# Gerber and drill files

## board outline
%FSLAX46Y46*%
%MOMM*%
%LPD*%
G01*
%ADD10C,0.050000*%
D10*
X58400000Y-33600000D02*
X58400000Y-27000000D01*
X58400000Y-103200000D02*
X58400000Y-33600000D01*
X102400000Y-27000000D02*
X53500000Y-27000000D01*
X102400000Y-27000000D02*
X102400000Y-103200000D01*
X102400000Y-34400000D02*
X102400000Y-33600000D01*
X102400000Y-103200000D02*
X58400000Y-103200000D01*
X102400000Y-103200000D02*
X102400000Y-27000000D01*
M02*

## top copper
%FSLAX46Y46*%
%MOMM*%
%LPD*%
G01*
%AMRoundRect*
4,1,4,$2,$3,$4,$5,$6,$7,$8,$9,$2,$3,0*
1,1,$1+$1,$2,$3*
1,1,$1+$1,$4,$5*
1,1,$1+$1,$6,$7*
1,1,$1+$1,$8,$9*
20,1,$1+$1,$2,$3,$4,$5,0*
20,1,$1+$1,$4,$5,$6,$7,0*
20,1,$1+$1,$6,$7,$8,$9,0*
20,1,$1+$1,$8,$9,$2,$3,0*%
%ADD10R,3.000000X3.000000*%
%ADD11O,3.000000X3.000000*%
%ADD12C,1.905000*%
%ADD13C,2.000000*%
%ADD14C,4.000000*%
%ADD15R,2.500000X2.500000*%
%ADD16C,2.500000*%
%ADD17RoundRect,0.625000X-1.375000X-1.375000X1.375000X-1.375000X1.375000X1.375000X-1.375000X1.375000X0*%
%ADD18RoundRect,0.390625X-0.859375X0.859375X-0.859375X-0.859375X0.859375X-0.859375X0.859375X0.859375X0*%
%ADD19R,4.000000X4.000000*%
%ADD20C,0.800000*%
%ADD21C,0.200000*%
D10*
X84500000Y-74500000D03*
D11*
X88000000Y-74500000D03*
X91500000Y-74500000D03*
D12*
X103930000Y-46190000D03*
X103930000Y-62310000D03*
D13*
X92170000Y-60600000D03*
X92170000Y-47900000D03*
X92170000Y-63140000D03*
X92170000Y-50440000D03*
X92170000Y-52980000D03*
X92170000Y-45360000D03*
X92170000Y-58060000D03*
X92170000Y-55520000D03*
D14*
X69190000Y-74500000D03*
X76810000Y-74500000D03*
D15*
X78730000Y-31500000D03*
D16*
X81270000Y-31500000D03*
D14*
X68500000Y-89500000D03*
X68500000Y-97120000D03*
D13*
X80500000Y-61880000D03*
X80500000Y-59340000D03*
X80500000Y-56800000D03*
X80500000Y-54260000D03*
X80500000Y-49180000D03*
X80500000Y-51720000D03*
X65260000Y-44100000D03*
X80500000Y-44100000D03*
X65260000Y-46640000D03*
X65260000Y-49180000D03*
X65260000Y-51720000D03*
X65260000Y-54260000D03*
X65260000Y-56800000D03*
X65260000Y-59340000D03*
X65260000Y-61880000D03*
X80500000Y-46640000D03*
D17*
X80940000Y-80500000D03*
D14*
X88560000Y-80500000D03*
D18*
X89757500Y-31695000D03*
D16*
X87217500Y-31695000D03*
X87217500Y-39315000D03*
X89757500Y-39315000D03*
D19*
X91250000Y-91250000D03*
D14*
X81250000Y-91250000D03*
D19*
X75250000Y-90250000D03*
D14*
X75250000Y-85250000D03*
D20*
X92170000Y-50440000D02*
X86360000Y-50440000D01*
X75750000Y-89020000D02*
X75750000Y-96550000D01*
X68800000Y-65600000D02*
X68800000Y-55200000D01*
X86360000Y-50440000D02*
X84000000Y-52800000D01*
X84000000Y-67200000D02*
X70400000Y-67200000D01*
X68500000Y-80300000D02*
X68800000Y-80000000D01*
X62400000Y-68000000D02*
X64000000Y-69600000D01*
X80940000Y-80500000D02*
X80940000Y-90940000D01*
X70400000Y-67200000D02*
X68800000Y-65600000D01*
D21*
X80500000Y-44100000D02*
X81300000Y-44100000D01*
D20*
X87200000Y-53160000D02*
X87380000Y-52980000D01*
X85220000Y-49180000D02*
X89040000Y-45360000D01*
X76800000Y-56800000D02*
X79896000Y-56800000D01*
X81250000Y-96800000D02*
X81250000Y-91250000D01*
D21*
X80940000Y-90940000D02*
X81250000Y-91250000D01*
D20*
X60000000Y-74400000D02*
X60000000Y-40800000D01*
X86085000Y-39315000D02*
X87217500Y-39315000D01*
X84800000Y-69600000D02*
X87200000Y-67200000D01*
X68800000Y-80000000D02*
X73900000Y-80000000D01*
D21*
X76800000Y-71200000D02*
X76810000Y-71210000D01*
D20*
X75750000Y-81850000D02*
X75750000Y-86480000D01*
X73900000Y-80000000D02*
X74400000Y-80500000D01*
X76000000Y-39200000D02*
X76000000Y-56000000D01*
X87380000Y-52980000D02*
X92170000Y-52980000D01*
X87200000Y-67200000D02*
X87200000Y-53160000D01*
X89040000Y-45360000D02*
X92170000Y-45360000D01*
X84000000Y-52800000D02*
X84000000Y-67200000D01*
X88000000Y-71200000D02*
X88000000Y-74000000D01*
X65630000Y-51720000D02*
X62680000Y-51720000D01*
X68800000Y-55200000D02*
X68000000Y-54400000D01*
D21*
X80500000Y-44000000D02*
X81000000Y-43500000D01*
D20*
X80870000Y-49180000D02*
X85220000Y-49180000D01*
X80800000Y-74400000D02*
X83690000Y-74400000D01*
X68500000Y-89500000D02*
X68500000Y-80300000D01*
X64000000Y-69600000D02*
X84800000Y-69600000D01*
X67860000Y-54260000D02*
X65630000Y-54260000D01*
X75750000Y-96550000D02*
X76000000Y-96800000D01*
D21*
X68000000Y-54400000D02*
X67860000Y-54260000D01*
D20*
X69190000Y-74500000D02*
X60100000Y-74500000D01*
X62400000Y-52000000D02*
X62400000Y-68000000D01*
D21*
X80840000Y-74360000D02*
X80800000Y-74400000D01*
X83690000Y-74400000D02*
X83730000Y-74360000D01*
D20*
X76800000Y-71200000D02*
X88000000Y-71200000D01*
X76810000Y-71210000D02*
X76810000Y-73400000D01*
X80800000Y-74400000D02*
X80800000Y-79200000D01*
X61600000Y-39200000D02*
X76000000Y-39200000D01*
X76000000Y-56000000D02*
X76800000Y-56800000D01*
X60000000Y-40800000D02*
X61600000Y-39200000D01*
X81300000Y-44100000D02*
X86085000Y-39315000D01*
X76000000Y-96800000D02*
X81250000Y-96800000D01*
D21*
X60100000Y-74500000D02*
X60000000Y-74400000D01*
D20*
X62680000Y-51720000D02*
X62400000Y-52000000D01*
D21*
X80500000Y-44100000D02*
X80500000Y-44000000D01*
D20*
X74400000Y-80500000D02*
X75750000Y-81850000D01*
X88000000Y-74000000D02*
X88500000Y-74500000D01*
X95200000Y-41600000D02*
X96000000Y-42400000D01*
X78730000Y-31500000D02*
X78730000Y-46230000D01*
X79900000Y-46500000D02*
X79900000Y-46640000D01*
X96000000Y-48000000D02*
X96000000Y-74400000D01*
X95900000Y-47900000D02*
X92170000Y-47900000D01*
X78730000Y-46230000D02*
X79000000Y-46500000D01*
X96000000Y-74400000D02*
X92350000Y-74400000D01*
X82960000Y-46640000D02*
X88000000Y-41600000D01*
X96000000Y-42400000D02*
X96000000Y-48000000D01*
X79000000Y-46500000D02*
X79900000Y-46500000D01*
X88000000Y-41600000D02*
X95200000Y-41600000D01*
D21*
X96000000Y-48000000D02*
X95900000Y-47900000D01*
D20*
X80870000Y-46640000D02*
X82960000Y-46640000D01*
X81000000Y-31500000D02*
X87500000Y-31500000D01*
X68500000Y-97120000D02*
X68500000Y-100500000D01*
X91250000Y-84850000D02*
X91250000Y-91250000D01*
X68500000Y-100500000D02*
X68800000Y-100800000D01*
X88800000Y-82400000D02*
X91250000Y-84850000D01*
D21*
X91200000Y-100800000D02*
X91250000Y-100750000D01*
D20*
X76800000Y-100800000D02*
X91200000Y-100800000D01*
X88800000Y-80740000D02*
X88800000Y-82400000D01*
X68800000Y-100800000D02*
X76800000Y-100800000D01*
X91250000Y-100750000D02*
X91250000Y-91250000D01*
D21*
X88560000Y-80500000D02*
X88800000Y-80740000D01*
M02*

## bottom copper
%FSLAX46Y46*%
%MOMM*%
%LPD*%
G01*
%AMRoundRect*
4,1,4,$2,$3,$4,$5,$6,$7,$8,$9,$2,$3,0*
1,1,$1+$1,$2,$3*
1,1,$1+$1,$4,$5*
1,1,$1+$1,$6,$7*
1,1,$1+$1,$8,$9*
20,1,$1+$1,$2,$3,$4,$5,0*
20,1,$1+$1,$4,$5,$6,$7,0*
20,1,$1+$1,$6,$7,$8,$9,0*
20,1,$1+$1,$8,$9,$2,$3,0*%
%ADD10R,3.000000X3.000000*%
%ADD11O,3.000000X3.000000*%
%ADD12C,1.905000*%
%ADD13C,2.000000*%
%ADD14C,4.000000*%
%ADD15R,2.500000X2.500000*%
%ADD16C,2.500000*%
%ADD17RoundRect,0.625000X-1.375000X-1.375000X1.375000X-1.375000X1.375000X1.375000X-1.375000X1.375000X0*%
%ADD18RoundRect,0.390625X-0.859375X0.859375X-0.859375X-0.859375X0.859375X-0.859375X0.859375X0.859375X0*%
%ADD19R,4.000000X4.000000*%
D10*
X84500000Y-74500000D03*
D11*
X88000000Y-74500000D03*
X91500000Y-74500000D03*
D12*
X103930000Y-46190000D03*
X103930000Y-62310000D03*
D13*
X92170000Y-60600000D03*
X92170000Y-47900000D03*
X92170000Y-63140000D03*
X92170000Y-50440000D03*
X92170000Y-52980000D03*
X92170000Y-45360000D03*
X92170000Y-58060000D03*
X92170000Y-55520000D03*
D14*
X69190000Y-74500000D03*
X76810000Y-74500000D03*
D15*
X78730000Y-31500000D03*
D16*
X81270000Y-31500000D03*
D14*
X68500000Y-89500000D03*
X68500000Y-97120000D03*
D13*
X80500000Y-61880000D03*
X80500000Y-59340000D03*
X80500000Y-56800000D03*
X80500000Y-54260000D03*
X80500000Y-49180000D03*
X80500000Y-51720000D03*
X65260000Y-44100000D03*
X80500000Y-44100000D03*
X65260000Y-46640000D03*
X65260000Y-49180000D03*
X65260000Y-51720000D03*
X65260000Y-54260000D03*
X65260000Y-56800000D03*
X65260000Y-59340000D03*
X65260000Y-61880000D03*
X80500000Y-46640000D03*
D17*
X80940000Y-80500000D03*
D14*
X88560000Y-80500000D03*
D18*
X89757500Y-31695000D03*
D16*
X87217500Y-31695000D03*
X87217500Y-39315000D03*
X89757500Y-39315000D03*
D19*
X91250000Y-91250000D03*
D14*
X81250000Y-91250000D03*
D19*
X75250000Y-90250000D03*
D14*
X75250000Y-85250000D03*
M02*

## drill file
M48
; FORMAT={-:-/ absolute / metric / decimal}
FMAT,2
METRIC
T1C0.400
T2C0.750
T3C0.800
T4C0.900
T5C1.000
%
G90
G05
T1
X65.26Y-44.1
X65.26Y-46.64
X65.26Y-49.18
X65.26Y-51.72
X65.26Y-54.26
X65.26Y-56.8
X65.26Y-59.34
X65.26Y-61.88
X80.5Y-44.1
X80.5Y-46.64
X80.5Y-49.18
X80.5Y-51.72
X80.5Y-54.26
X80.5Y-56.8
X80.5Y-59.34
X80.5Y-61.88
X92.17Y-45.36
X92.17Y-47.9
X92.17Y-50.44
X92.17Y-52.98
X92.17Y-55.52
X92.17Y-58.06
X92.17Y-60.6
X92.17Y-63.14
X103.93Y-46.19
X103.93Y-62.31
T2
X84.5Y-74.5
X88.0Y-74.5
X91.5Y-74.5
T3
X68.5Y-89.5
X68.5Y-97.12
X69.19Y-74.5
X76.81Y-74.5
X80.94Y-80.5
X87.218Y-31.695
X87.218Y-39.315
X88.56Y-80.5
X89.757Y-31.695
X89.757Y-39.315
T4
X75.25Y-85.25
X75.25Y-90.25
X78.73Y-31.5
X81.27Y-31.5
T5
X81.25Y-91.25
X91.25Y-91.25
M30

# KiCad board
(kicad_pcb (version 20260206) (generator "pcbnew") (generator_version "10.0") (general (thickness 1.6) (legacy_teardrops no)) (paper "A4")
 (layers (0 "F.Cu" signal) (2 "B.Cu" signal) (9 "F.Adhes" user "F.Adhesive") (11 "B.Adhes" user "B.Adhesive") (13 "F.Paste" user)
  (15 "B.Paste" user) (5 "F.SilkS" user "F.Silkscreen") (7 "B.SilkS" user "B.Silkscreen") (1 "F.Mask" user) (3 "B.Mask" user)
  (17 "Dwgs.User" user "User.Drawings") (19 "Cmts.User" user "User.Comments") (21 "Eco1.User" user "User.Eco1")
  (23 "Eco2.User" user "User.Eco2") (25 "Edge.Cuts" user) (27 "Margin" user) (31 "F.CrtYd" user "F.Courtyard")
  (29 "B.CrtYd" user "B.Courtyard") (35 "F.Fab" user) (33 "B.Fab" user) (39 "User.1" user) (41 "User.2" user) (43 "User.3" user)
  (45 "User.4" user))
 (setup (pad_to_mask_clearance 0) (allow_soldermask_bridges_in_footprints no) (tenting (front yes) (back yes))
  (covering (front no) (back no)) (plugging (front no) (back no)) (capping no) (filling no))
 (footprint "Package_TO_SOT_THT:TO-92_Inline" (layer "F.Cu") (at 87 74.5)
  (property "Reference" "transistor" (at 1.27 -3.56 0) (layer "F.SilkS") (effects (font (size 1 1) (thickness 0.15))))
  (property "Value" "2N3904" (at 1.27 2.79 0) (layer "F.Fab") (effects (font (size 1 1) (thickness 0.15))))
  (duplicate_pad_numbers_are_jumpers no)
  (pad "1" thru_hole rect (at -2.5 0) (size 3 3) (drill 0.75) (layers "*.Cu" "*.Mask") (remove_unused_layers no))
  (pad "2" thru_hole oval (at 1 0) (size 3 3) (drill 0.75) (layers "*.Cu" "*.Mask") (remove_unused_layers no))
  (pad "3" thru_hole oval (at 4.5 0) (size 3 3) (drill 0.75) (layers "*.Cu" "*.Mask") (remove_unused_layers no)))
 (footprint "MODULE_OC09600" (layer "F.Cu") (at 98.5 54.25)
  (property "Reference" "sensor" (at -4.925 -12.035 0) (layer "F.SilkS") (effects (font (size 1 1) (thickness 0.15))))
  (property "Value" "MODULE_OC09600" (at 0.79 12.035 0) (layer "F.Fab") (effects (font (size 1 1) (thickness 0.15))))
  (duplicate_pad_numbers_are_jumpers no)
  (pad "" thru_hole circle (at 5.43 -8.06) (size 1.905 1.905) (drill 0.4) (layers "*.Cu" "*.Mask") (remove_unused_layers no)
   (solder_mask_margin 0.102))
  (pad "" thru_hole circle (at 5.43 8.06) (size 1.905 1.905) (drill 0.4) (layers "*.Cu" "*.Mask") (remove_unused_layers no)
   (solder_mask_margin 0.102))
  (pad "AD0" thru_hole circle (at -6.33 6.35) (size 2 1.905) (drill 0.4) (layers "*.Cu" "*.Mask") (remove_unused_layers no)
   (solder_mask_margin 0.102))
  (pad "GND" thru_hole circle (at -6.33 -6.35) (size 2 1.905) (drill 0.4) (layers "*.Cu" "*.Mask") (remove_unused_layers no)
   (solder_mask_margin 0.102))
  (pad "INT" thru_hole circle (at -6.33 8.89) (size 2 1.905) (drill 0.4) (layers "*.Cu" "*.Mask") (remove_unused_layers no)
   (solder_mask_margin 0.102))
  (pad "SCL" thru_hole circle (at -6.33 -3.81) (size 2 1.905) (drill 0.4) (layers "*.Cu" "*.Mask") (remove_unused_layers no)
   (solder_mask_margin 0.102))
  (pad "SDA" thru_hole circle (at -6.33 -1.27) (size 2 1.905) (drill 0.4) (layers "*.Cu" "*.Mask") (remove_unused_layers no)
   (solder_mask_margin 0.102))
  (pad "VCC" thru_hole circle (at -6.33 -8.89) (size 2 2) (drill 0.4) (layers "*.Cu" "*.Mask") (remove_unused_layers no)
   (solder_mask_margin 0.102))
  (pad "XCL" thru_hole circle (at -6.33 3.81) (size 2 1.905) (drill 0.4) (layers "*.Cu" "*.Mask") (remove_unused_layers no)
   (solder_mask_margin 0.102))
  (pad "XDA" thru_hole circle (at -6.33 1.27) (size 2 1.905) (drill 0.4) (layers "*.Cu" "*.Mask") (remove_unused_layers no)
   (solder_mask_margin 0.102)))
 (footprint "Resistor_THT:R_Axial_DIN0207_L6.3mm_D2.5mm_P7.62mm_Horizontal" (layer "F.Cu") (at 69.19 74.5)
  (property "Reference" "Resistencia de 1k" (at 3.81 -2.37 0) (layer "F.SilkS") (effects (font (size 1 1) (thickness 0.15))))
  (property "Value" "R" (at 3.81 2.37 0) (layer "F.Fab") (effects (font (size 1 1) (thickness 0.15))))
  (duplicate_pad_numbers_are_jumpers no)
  (pad "1" thru_hole circle (at 0 0) (size 4 1.6) (drill 0.8) (layers "*.Cu" "*.Mask") (remove_unused_layers no))
  (pad "2" thru_hole circle (at 7.62 0) (size 4 1.6) (drill 0.8) (layers "*.Cu" "*.Mask") (remove_unused_layers no)))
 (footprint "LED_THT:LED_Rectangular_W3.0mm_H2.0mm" (layer "F.Cu") (at 78.73 31.5)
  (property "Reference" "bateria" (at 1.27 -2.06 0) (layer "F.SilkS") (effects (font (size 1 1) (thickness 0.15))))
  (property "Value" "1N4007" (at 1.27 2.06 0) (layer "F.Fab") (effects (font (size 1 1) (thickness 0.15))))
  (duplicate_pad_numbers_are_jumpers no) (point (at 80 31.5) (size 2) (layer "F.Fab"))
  (pad "1" thru_hole rect (at 0 0) (size 2.5 2.5) (drill 0.9) (layers "*.Cu" "*.Mask") (remove_unused_layers no)
   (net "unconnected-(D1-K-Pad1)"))
  (pad "2" thru_hole circle (at 2.54 0) (size 2.5 1.8) (drill 0.9) (layers "*.Cu" "*.Mask") (remove_unused_layers no)
   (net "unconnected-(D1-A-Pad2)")))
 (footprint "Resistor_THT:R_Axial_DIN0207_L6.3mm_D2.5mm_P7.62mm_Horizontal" (layer "F.Cu") (at 68.5 89.5 -90)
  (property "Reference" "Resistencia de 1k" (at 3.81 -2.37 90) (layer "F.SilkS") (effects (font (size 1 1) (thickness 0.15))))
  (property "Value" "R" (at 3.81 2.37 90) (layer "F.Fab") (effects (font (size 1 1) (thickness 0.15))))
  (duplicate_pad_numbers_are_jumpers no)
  (pad "1" thru_hole circle (at 0 0 270) (size 4 1.6) (drill 0.8) (layers "*.Cu" "*.Mask") (remove_unused_layers no))
  (pad "2" thru_hole circle (at 7.62 0 270) (size 4 1.6) (drill 0.8) (layers "*.Cu" "*.Mask") (remove_unused_layers no)))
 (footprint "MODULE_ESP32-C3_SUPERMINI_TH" (layer "F.Cu") (at 72.88 54)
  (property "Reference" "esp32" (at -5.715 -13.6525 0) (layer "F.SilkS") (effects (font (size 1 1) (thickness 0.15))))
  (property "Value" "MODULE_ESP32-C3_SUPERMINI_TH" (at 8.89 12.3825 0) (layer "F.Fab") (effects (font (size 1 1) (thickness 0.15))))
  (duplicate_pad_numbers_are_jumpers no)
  (pad "0" thru_hole circle (at 7.62 7.88) (size 2 2) (drill 0.4) (layers "*.Cu" "*.Mask") (remove_unused_layers no)
   (solder_mask_margin 0.102))
  (pad "1" thru_hole circle (at 7.62 5.34) (size 2 2) (drill 0.4) (layers "*.Cu" "*.Mask") (remove_unused_layers no)
   (solder_mask_margin 0.102))
  (pad "2" thru_hole circle (at 7.62 2.8) (size 2 2) (drill 0.4) (layers "*.Cu" "*.Mask") (remove_unused_layers no)
   (solder_mask_margin 0.102))
  (pad "3" thru_hole circle (at 7.62 0.26) (size 2 2) (drill 0.4) (layers "*.Cu" "*.Mask") (remove_unused_layers no)
   (solder_mask_margin 0.102))
  (pad "3.3" thru_hole circle (at 7.62 -4.82) (size 2 2) (drill 0.4) (layers "*.Cu" "*.Mask") (remove_unused_layers no)
   (solder_mask_margin 0.102))
  (pad "4" thru_hole circle (at 7.62 -2.28) (size 2 2) (drill 0.4) (layers "*.Cu" "*.Mask") (remove_unused_layers no)
   (solder_mask_margin 0.102))
  (pad "5" thru_hole circle (at -7.62 -9.9) (size 2 2) (drill 0.4) (layers "*.Cu" "*.Mask") (remove_unused_layers no)
   (solder_mask_margin 0.102))
  (pad "5V" thru_hole circle (at 7.62 -9.9) (size 2 2) (drill 0.4) (layers "*.Cu" "*.Mask") (remove_unused_layers no)
   (solder_mask_margin 0.102))
  (pad "6" thru_hole circle (at -7.62 -7.36) (size 2 2) (drill 0.4) (layers "*.Cu" "*.Mask") (remove_unused_layers no)
   (solder_mask_margin 0.102))
  (pad "7" thru_hole circle (at -7.62 -4.82) (size 2 2) (drill 0.4) (layers "*.Cu" "*.Mask") (remove_unused_layers no)
   (solder_mask_margin 0.102))
  (pad "8" thru_hole circle (at -7.62 -2.28) (size 2 2) (drill 0.4) (layers "*.Cu" "*.Mask") (remove_unused_layers no)
   (solder_mask_margin 0.102))
  (pad "9" thru_hole circle (at -7.62 0.26) (size 2 2) (drill 0.4) (layers "*.Cu" "*.Mask") (remove_unused_layers no)
   (solder_mask_margin 0.102))
  (pad "10" thru_hole circle (at -7.62 2.8) (size 2 2) (drill 0.4) (layers "*.Cu" "*.Mask") (remove_unused_layers no)
   (solder_mask_margin 0.102))
  (pad "20" thru_hole circle (at -7.62 5.34) (size 2 2) (drill 0.4) (layers "*.Cu" "*.Mask") (remove_unused_layers no)
   (solder_mask_margin 0.102))
  (pad "21" thru_hole circle (at -7.62 7.88) (size 2 2) (drill 0.4) (layers "*.Cu" "*.Mask") (remove_unused_layers no)
   (solder_mask_margin 0.102))
  (pad "G" thru_hole circle (at 7.62 -7.36) (size 2 2) (drill 0.4) (layers "*.Cu" "*.Mask") (remove_unused_layers no)
   (solder_mask_margin 0.102)))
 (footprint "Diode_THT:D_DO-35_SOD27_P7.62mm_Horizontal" (layer "F.Cu") (at 80.94 80.5)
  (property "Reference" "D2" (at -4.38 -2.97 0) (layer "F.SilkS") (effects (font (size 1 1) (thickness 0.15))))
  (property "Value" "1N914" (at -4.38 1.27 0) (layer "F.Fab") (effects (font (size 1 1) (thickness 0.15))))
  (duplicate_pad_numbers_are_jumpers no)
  (pad "1" thru_hole roundrect (at 0 0) (size 4 4) (drill 0.8) (layers "*.Cu" "*.Mask") (remove_unused_layers no) (roundrect_rratio 0.15625))
  (pad "2" thru_hole circle (at 7.62 0) (size 4 1.6) (drill 0.8) (layers "*.Cu" "*.Mask") (remove_unused_layers no)))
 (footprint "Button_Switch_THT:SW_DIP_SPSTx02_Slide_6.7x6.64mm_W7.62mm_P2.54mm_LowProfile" (layer "F.Cu") (at 89.7575 31.695 -90)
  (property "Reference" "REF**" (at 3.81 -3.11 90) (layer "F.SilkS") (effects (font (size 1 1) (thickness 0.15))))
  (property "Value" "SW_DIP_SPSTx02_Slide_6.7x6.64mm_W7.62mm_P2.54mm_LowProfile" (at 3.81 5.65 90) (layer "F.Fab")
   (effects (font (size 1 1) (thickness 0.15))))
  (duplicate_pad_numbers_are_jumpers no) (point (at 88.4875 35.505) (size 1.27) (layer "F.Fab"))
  (pad "1" thru_hole roundrect (at 0 0 270) (size 2.5 2.5) (drill 0.8) (layers "*.Cu" "*.Mask") (remove_unused_layers no)
   (roundrect_rratio 0.15625))
  (pad "2" thru_hole circle (at 0 2.54 270) (size 2.5 2.5) (drill 0.8) (layers "*.Cu" "*.Mask") (remove_unused_layers no))
  (pad "3" thru_hole circle (at 7.62 2.54 270) (size 2.5 2) (drill 0.8) (layers "*.Cu" "*.Mask") (remove_unused_layers no))
  (pad "4" thru_hole circle (at 7.62 0 270) (size 2.5 2) (drill 0.8) (layers "*.Cu" "*.Mask") (remove_unused_layers no)))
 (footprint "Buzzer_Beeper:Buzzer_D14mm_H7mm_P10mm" (layer "F.Cu") (at 91.25 91.25 180)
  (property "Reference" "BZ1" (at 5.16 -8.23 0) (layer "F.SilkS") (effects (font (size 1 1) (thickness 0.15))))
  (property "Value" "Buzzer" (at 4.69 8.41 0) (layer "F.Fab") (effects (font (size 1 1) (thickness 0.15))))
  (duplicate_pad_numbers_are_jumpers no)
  (pad "1" thru_hole rect (at 0 0 180) (size 4 4) (drill 1) (layers "*.Cu" "*.Mask") (remove_unused_layers no))
  (pad "2" thru_hole circle (at 10 0 180) (size 4 2) (drill 1) (layers "*.Cu" "*.Mask") (remove_unused_layers no)))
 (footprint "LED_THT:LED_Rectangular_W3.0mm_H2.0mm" (layer "F.Cu") (at 75.25 89.75 90)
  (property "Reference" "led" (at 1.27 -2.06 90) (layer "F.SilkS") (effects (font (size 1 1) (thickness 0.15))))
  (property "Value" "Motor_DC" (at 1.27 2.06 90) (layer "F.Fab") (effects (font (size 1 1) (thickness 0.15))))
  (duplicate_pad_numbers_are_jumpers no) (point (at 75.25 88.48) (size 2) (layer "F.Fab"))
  (pad "1" thru_hole rect (at -0.5 0 90) (size 4 4) (drill 0.9) (layers "*.Cu" "*.Mask") (remove_unused_layers no))
  (pad "2" thru_hole circle (at 4.5 0 90) (size 4 4) (drill 0.9) (layers "*.Cu" "*.Mask") (remove_unused_layers no)))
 (gr_line (start 58.4 33.6) (end 58.4 27) (stroke (width 0.05) (type default)) (layer "Edge.Cuts"))
 (gr_line (start 58.4 103.2) (end 58.4 33.6) (stroke (width 0.05) (type default)) (layer "Edge.Cuts"))
 (gr_line (start 102.4 27) (end 53.5 27) (stroke (width 0.05) (type default)) (layer "Edge.Cuts"))
 (gr_line (start 102.4 27) (end 102.4 103.2) (stroke (width 0.05) (type default)) (layer "Edge.Cuts"))
 (gr_line (start 102.4 34.4) (end 102.4 33.6) (stroke (width 0.05) (type default)) (layer "Edge.Cuts"))
 (gr_line (start 102.4 103.2) (end 58.4 103.2) (stroke (width 0.05) (type default)) (layer "Edge.Cuts"))
 (gr_line (start 102.4 103.2) (end 102.4 27) (stroke (width 0.05) (type default)) (layer "Edge.Cuts"))
 (segment (start 92.17 50.44) (end 86.36 50.44) (width 0.8) (layer "F.Cu") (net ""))
 (segment (start 75.75 89.02) (end 75.75 96.55) (width 0.8) (layer "F.Cu") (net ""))
 (segment (start 68.8 65.6) (end 68.8 55.2) (width 0.8) (layer "F.Cu") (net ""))
 (segment (start 86.36 50.44) (end 84 52.8) (width 0.8) (layer "F.Cu") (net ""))
 (segment (start 84 67.2) (end 70.4 67.2) (width 0.8) (layer "F.Cu") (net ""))
 (segment (start 68.5 80.3) (end 68.8 80) (width 0.8) (layer "F.Cu") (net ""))
 (segment (start 62.4 68) (end 64 69.6) (width 0.8) (layer "F.Cu") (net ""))
 (segment (start 80.94 80.5) (end 80.94 90.94) (width 0.8) (layer "F.Cu") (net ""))
 (segment (start 70.4 67.2) (end 68.8 65.6) (width 0.8) (layer "F.Cu") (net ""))
 (segment (start 80.5 44.1) (end 81.3 44.1) (width 0.2) (layer "F.Cu") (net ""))
 (segment (start 87.2 53.16) (end 87.38 52.98) (width 0.8) (layer "F.Cu") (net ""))
 (segment (start 85.22 49.18) (end 89.04 45.36) (width 0.8) (layer "F.Cu") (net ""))
 (segment (start 76.8 56.8) (end 79.896 56.8) (width 0.8) (layer "F.Cu") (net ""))
 (segment (start 81.25 96.8) (end 81.25 91.25) (width 0.8) (layer "F.Cu") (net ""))
 (segment (start 80.94 90.94) (end 81.25 91.25) (width 0.2) (layer "F.Cu") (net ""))
 (segment (start 60 74.4) (end 60 40.8) (width 0.8) (layer "F.Cu") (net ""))
 (segment (start 86.085 39.315) (end 87.2175 39.315) (width 0.8) (layer "F.Cu") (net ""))
 (segment (start 84.8 69.6) (end 87.2 67.2) (width 0.8) (layer "F.Cu") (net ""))
 (segment (start 68.8 80) (end 73.9 80) (width 0.8) (layer "F.Cu") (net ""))
 (segment (start 76.8 71.2) (end 76.81 71.21) (width 0.2) (layer "F.Cu") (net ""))
 (segment (start 75.75 81.85) (end 75.75 86.48) (width 0.8) (layer "F.Cu") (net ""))
 (segment (start 73.9 80) (end 74.4 80.5) (width 0.8) (layer "F.Cu") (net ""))
 (segment (start 76 39.2) (end 76 56) (width 0.8) (layer "F.Cu") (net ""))
 (segment (start 87.38 52.98) (end 92.17 52.98) (width 0.8) (layer "F.Cu") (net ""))
 (segment (start 87.2 67.2) (end 87.2 53.16) (width 0.8) (layer "F.Cu") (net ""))
 (segment (start 89.04 45.36) (end 92.17 45.36) (width 0.8) (layer "F.Cu") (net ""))
 (segment (start 84 52.8) (end 84 67.2) (width 0.8) (layer "F.Cu") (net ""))
 (segment (start 88 71.2) (end 88 74) (width 0.8) (layer "F.Cu") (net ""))
 (segment (start 65.63 51.72) (end 62.68 51.72) (width 0.8) (layer "F.Cu") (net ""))
 (segment (start 68.8 55.2) (end 68 54.4) (width 0.8) (layer "F.Cu") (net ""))
 (segment (start 80.5 44) (end 81 43.5) (width 0.2) (layer "F.Cu") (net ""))
 (segment (start 80.87 49.18) (end 85.22 49.18) (width 0.8) (layer "F.Cu") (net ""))
 (segment (start 80.8 74.4) (end 83.69 74.4) (width 0.8) (layer "F.Cu") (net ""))
 (segment (start 68.5 89.5) (end 68.5 80.3) (width 0.8) (layer "F.Cu") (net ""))
 (segment (start 64 69.6) (end 84.8 69.6) (width 0.8) (layer "F.Cu") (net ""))
 (segment (start 67.86 54.26) (end 65.63 54.26) (width 0.8) (layer "F.Cu") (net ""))
 (segment (start 75.75 96.55) (end 76 96.8) (width 0.8) (layer "F.Cu") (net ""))
 (segment (start 68 54.4) (end 67.86 54.26) (width 0.2) (layer "F.Cu") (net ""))
 (segment (start 69.19 74.5) (end 60.1 74.5) (width 0.8) (layer "F.Cu") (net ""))
 (segment (start 62.4 52) (end 62.4 68) (width 0.8) (layer "F.Cu") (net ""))
 (segment (start 80.84 74.36) (end 80.8 74.4) (width 0.2) (layer "F.Cu") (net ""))
 (segment (start 83.69 74.4) (end 83.73 74.36) (width 0.2) (layer "F.Cu") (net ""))
 (segment (start 76.8 71.2) (end 88 71.2) (width 0.8) (layer "F.Cu") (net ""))
 (segment (start 76.81 71.21) (end 76.81 73.4) (width 0.8) (layer "F.Cu") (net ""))
 (segment (start 80.8 74.4) (end 80.8 79.2) (width 0.8) (layer "F.Cu") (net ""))
 (segment (start 61.6 39.2) (end 76 39.2) (width 0.8) (layer "F.Cu") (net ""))
 (segment (start 76 56) (end 76.8 56.8) (width 0.8) (layer "F.Cu") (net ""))
 (segment (start 60 40.8) (end 61.6 39.2) (width 0.8) (layer "F.Cu") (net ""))
 (segment (start 81.3 44.1) (end 86.085 39.315) (width 0.8) (layer "F.Cu") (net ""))
 (segment (start 76 96.8) (end 81.25 96.8) (width 0.8) (layer "F.Cu") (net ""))
 (segment (start 60.1 74.5) (end 60 74.4) (width 0.2) (layer "F.Cu") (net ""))
 (segment (start 62.68 51.72) (end 62.4 52) (width 0.8) (layer "F.Cu") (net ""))
 (segment (start 80.5 44.1) (end 80.5 44) (width 0.2) (layer "F.Cu") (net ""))
 (segment (start 74.4 80.5) (end 75.75 81.85) (width 0.8) (layer "F.Cu") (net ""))
 (segment (start 88 74) (end 88.5 74.5) (width 0.8) (layer "F.Cu") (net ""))
 (segment (start 95.2 41.6) (end 96 42.4) (width 0.8) (layer "F.Cu") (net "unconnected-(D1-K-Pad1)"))
 (segment (start 78.73 31.5) (end 78.73 46.23) (width 0.8) (layer "F.Cu") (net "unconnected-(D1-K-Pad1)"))
 (segment (start 79.9 46.5) (end 79.9 46.64) (width 0.8) (layer "F.Cu") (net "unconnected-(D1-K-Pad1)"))
 (segment (start 96 48) (end 96 74.4) (width 0.8) (layer "F.Cu") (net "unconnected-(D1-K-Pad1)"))
 (segment (start 95.9 47.9) (end 92.17 47.9) (width 0.8) (layer "F.Cu") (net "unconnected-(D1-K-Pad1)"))
 (segment (start 78.73 46.23) (end 79 46.5) (width 0.8) (layer "F.Cu") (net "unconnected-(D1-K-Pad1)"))
 (segment (start 96 74.4) (end 92.35 74.4) (width 0.8) (layer "F.Cu") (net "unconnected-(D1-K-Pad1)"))
 (segment (start 82.96 46.64) (end 88 41.6) (width 0.8) (layer "F.Cu") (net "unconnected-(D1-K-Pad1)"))
 (segment (start 96 42.4) (end 96 48) (width 0.8) (layer "F.Cu") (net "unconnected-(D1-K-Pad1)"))
 (segment (start 79 46.5) (end 79.9 46.5) (width 0.8) (layer "F.Cu") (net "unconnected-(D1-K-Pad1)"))
 (segment (start 88 41.6) (end 95.2 41.6) (width 0.8) (layer "F.Cu") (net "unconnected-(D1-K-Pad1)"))
 (segment (start 96 48) (end 95.9 47.9) (width 0.2) (layer "F.Cu") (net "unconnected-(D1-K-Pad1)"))
 (segment (start 80.87 46.64) (end 82.96 46.64) (width 0.8) (layer "F.Cu") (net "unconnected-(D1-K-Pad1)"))
 (segment (start 81 31.5) (end 87.5 31.5) (width 0.8) (layer "F.Cu") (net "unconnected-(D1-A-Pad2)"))
 (segment (start 68.5 97.12) (end 68.5 100.5) (width 0.8) (layer "F.Cu") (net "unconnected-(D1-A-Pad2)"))
 (segment (start 91.25 84.85) (end 91.25 91.25) (width 0.8) (layer "F.Cu") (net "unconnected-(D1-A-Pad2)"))
 (segment (start 68.5 100.5) (end 68.8 100.8) (width 0.8) (layer "F.Cu") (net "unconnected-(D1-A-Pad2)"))
 (segment (start 88.8 82.4) (end 91.25 84.85) (width 0.8) (layer "F.Cu") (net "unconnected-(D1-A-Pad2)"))
 (segment (start 91.2 100.8) (end 91.25 100.75) (width 0.2) (layer "F.Cu") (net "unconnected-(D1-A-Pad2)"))
 (segment (start 76.8 100.8) (end 91.2 100.8) (width 0.8) (layer "F.Cu") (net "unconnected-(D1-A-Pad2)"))
 (segment (start 88.8 80.74) (end 88.8 82.4) (width 0.8) (layer "F.Cu") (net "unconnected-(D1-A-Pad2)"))
 (segment (start 68.8 100.8) (end 76.8 100.8) (width 0.8) (layer "F.Cu") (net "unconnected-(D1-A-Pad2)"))
 (segment (start 91.25 100.75) (end 91.25 91.25) (width 0.8) (layer "F.Cu") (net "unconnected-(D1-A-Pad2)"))
 (segment (start 88.56 80.5) (end 88.8 80.74) (width 0.2) (layer "F.Cu") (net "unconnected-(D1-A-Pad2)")))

